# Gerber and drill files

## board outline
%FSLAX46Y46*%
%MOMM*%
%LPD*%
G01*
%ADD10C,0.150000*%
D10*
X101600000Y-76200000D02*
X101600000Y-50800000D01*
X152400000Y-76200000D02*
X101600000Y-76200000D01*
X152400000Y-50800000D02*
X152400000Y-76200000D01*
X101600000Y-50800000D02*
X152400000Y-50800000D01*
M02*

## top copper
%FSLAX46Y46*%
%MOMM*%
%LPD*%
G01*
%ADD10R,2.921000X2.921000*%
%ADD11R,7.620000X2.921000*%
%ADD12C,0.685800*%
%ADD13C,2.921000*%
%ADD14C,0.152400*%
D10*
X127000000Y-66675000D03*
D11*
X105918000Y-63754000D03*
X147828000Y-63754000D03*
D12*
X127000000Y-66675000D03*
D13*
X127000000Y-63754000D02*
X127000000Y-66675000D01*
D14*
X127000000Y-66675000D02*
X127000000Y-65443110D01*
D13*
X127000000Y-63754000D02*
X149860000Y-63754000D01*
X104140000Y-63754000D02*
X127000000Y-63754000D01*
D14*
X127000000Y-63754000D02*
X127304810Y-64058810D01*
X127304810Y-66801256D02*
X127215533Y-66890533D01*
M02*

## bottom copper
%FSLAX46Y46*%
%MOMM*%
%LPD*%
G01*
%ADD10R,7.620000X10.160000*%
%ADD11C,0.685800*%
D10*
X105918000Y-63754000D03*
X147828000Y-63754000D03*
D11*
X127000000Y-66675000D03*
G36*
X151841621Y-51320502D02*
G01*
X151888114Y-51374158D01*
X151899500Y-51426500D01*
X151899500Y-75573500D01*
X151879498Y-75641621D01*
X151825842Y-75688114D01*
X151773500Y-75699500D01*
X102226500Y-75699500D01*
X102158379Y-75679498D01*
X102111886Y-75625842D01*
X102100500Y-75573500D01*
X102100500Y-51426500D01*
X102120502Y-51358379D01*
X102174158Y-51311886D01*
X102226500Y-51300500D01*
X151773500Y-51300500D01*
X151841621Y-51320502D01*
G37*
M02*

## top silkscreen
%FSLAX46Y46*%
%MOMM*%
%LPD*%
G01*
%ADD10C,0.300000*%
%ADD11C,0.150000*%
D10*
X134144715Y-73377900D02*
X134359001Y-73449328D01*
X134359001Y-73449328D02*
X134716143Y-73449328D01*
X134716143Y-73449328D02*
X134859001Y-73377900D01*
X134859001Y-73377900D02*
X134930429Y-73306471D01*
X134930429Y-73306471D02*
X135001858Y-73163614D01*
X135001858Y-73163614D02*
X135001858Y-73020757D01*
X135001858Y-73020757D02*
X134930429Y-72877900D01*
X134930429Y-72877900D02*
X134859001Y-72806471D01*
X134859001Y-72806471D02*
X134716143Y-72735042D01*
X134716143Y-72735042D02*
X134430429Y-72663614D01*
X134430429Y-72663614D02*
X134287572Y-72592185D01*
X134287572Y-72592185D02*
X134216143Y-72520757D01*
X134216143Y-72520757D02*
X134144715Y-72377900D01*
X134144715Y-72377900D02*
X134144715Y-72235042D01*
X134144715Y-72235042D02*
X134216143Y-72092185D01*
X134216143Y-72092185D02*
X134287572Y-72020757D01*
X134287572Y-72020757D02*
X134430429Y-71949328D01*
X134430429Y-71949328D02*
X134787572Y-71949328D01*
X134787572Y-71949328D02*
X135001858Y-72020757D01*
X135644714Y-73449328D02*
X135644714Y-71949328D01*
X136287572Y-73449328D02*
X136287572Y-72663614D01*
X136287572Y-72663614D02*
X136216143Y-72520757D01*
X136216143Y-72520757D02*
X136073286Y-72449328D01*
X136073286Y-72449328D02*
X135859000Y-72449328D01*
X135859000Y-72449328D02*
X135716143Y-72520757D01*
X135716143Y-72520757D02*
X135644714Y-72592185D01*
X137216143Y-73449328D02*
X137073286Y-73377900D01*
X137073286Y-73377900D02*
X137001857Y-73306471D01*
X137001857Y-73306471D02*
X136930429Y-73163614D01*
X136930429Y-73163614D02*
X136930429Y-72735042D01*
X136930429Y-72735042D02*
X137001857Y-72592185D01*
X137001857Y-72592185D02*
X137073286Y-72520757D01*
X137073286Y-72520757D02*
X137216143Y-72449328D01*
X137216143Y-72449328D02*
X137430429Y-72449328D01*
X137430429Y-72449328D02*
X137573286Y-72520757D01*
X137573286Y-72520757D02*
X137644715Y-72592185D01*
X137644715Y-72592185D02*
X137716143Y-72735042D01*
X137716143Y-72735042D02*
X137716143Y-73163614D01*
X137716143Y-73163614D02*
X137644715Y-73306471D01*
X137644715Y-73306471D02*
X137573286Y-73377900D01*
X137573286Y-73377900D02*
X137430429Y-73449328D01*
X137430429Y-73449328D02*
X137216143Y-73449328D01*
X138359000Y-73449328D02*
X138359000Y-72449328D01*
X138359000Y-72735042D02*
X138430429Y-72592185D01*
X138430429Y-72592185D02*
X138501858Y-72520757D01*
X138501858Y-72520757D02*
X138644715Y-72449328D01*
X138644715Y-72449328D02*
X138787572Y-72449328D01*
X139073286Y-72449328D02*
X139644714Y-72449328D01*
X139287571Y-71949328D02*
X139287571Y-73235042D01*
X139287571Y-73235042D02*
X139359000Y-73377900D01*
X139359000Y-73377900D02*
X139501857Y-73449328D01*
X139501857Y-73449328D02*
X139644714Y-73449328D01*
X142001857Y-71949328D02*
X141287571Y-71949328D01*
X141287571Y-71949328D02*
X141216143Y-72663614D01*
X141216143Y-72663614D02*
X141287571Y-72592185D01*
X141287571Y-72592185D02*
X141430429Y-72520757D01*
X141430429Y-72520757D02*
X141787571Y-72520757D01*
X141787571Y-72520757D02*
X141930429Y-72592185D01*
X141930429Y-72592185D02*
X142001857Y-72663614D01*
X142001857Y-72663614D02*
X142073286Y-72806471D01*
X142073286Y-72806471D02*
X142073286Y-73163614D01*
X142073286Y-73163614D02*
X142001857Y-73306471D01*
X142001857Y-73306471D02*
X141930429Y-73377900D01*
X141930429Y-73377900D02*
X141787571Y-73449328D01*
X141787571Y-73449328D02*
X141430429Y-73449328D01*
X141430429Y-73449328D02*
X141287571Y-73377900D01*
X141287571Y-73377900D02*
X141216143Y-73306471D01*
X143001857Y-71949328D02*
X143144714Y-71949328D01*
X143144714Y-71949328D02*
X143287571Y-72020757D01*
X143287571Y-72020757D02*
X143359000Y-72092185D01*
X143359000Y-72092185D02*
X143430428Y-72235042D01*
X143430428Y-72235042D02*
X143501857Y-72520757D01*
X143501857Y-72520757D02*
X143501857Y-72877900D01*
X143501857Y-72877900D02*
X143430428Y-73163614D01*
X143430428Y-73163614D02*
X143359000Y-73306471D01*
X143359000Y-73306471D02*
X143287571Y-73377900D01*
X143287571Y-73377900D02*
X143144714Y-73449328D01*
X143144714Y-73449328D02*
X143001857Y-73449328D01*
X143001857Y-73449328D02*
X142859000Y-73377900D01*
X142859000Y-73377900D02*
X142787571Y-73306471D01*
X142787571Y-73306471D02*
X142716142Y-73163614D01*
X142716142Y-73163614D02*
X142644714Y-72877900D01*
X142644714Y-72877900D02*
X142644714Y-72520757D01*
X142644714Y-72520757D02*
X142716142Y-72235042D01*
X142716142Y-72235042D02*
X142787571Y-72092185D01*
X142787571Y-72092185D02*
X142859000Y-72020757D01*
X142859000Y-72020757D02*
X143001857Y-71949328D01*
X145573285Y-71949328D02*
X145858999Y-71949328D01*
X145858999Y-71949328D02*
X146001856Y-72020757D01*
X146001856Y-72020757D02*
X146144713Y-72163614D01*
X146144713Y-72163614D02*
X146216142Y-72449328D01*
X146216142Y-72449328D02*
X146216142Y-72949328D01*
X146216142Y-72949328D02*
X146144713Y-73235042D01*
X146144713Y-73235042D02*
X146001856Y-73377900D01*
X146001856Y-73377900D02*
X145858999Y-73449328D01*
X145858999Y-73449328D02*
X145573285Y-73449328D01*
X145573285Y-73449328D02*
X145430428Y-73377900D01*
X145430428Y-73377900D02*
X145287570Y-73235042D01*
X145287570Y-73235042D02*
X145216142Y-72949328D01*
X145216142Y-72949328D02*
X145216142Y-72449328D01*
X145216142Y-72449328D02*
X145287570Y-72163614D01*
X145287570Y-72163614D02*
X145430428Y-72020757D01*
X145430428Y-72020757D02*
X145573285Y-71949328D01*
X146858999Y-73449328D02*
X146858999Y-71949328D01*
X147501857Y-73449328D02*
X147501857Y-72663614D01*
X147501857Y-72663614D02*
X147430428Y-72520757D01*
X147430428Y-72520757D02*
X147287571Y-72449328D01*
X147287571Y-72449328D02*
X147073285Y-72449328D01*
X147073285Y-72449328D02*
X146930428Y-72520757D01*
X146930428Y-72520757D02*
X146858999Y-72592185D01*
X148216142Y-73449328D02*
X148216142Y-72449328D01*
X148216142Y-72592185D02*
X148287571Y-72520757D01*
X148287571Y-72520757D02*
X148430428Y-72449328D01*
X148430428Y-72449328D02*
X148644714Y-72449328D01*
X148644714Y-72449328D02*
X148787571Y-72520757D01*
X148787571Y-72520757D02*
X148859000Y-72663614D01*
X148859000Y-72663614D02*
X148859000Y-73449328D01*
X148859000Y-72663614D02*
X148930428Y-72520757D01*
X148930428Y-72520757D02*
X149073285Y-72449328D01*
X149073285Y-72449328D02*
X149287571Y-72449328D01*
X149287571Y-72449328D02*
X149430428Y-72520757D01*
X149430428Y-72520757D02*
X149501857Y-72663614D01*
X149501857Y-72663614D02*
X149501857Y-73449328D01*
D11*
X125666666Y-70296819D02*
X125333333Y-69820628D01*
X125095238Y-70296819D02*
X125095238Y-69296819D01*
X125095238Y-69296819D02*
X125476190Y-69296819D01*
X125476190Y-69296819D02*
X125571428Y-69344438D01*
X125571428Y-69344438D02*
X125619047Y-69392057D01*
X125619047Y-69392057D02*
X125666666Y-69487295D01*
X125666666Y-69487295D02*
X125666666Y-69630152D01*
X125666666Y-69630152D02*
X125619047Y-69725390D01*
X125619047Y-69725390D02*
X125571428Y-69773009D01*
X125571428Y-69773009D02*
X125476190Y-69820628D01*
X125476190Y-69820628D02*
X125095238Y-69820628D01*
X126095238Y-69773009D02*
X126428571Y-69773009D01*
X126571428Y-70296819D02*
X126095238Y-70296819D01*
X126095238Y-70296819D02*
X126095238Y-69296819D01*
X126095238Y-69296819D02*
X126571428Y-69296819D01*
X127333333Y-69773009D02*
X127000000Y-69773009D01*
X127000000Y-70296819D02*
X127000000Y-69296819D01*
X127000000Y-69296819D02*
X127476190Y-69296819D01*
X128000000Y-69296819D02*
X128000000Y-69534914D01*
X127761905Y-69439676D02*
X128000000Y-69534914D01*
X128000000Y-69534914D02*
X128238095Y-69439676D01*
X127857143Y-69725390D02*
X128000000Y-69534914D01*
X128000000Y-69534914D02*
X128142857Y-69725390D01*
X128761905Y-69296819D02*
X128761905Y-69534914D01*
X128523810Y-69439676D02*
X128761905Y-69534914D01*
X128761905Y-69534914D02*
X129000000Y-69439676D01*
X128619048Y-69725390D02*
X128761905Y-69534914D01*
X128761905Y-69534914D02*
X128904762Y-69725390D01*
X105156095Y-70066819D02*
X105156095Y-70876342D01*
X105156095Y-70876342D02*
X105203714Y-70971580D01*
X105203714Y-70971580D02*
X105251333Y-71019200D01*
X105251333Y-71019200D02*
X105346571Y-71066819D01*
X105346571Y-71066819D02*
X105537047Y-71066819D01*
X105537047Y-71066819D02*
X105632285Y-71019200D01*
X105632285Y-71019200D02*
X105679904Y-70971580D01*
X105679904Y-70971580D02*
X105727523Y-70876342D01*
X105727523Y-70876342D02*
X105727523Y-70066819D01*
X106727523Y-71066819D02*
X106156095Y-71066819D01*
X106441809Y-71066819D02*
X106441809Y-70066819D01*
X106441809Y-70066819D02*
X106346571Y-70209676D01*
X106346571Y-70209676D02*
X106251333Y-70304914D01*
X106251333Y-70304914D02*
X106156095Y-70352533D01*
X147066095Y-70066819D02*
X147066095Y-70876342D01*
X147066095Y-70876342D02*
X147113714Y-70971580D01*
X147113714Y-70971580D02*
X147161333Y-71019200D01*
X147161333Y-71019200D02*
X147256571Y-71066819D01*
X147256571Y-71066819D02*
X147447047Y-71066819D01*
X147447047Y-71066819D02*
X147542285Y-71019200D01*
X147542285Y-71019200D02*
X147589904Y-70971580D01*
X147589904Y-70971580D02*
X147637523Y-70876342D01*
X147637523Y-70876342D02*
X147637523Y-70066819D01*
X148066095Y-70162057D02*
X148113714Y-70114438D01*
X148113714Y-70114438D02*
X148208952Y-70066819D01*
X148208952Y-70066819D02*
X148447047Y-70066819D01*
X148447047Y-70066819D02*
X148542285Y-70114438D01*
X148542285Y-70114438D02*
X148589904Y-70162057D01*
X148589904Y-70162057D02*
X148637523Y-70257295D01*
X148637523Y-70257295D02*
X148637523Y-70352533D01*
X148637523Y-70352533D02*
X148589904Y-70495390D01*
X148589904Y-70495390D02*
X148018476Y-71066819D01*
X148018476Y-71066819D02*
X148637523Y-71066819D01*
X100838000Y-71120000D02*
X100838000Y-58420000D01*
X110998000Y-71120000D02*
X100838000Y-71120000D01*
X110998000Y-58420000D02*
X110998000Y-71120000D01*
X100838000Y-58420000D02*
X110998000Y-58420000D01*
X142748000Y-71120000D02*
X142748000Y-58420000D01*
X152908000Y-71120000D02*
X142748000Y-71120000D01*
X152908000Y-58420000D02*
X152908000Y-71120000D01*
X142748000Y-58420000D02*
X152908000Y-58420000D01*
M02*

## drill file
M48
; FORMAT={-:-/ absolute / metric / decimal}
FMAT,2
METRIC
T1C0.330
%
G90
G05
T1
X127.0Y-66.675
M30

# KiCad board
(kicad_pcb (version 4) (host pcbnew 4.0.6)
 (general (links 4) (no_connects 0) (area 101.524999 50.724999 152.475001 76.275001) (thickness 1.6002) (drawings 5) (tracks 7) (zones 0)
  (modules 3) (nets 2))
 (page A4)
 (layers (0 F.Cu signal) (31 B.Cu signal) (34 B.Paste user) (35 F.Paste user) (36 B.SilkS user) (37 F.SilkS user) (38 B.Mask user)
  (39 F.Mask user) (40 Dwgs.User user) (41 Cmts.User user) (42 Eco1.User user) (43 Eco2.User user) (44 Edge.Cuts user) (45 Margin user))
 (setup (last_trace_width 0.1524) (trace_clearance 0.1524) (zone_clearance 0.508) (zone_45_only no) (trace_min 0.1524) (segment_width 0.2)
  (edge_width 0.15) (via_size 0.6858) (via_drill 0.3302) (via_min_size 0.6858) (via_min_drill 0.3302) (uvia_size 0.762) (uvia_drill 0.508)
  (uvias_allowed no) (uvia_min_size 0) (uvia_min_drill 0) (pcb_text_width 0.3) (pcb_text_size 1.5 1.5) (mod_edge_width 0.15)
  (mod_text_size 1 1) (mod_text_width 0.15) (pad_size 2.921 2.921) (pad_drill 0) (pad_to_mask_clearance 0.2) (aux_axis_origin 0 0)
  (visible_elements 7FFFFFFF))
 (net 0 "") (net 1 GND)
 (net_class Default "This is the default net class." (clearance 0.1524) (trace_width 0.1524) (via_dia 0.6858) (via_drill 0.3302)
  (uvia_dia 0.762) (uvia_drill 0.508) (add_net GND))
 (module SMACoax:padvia (layer F.Cu) (at 127 69.342)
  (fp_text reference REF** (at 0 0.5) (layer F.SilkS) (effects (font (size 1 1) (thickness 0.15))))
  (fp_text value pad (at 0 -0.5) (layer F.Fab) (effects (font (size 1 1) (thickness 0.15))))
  (pad 1 smd rect (at 0 -2.667) (size 2.921 2.921) (layers F.Cu F.Paste F.Mask) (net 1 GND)))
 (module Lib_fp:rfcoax (layer F.Cu) (at 107.188 66.04)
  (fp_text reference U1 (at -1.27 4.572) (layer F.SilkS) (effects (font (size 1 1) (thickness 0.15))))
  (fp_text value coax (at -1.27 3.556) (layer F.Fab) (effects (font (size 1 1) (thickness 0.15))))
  (fp_line (start -6.35 5.08) (end -6.35 -7.62) (layer F.SilkS) (width 0.15))
  (fp_line (start 3.81 5.08) (end -6.35 5.08) (layer F.SilkS) (width 0.15))
  (fp_line (start 3.81 -7.62) (end 3.81 5.08) (layer F.SilkS) (width 0.15))
  (fp_line (start -6.35 -7.62) (end 3.81 -7.62) (layer F.SilkS) (width 0.15))
  (pad 1 smd rect (at -1.27 -2.286) (size 7.62 2.921) (layers F.Cu F.Paste F.Mask) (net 1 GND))
  (pad 2 smd rect (at -1.27 -2.286) (size 7.62 10.16) (layers B.Cu B.Paste B.Mask) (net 1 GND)))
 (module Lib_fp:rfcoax (layer F.Cu) (at 149.098 66.04)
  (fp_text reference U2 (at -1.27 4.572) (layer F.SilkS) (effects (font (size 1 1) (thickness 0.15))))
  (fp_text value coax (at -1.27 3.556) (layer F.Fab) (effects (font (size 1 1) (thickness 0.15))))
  (fp_line (start -6.35 5.08) (end -6.35 -7.62) (layer F.SilkS) (width 0.15))
  (fp_line (start 3.81 5.08) (end -6.35 5.08) (layer F.SilkS) (width 0.15))
  (fp_line (start 3.81 -7.62) (end 3.81 5.08) (layer F.SilkS) (width 0.15))
  (fp_line (start -6.35 -7.62) (end 3.81 -7.62) (layer F.SilkS) (width 0.15))
  (pad 1 smd rect (at -1.27 -2.286) (size 7.62 2.921) (layers F.Cu F.Paste F.Mask) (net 1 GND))
  (pad 2 smd rect (at -1.27 -2.286) (size 7.62 10.16) (layers B.Cu B.Paste B.Mask) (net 1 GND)))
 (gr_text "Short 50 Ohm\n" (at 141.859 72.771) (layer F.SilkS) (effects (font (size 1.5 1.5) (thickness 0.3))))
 (gr_line (start 101.6 76.2) (end 101.6 50.8) (layer Edge.Cuts) (width 0.15))
 (gr_line (start 152.4 76.2) (end 101.6 76.2) (layer Edge.Cuts) (width 0.15))
 (gr_line (start 152.4 50.8) (end 152.4 76.2) (layer Edge.Cuts) (width 0.15))
 (gr_line (start 101.6 50.8) (end 152.4 50.8) (layer Edge.Cuts) (width 0.15))
 (segment (start 127 63.754) (end 127 66.675) (width 2.921) (layer F.Cu) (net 1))
 (via (at 127 66.675) (size 0.6858) (drill 0.3302) (layers F.Cu B.Cu) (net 1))
 (segment (start 127 66.675) (end 127 65.44311) (width 0.1524) (layer F.Cu) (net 1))
 (segment (start 127 63.754) (end 149.86 63.754) (width 2.921) (layer F.Cu) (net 1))
 (segment (start 104.14 63.754) (end 127 63.754) (width 2.921) (layer F.Cu) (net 1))
 (segment (start 127 63.754) (end 127.30481 64.05881) (width 0.1524) (layer F.Cu) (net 1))
 (segment (start 127.30481 66.801256) (end 127.215533 66.890533) (width 0.1524) (layer F.Cu) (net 1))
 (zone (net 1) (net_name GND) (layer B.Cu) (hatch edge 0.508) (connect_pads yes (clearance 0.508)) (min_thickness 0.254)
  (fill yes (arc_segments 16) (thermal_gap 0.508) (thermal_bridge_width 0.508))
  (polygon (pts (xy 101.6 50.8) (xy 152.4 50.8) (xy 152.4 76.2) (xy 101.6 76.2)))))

